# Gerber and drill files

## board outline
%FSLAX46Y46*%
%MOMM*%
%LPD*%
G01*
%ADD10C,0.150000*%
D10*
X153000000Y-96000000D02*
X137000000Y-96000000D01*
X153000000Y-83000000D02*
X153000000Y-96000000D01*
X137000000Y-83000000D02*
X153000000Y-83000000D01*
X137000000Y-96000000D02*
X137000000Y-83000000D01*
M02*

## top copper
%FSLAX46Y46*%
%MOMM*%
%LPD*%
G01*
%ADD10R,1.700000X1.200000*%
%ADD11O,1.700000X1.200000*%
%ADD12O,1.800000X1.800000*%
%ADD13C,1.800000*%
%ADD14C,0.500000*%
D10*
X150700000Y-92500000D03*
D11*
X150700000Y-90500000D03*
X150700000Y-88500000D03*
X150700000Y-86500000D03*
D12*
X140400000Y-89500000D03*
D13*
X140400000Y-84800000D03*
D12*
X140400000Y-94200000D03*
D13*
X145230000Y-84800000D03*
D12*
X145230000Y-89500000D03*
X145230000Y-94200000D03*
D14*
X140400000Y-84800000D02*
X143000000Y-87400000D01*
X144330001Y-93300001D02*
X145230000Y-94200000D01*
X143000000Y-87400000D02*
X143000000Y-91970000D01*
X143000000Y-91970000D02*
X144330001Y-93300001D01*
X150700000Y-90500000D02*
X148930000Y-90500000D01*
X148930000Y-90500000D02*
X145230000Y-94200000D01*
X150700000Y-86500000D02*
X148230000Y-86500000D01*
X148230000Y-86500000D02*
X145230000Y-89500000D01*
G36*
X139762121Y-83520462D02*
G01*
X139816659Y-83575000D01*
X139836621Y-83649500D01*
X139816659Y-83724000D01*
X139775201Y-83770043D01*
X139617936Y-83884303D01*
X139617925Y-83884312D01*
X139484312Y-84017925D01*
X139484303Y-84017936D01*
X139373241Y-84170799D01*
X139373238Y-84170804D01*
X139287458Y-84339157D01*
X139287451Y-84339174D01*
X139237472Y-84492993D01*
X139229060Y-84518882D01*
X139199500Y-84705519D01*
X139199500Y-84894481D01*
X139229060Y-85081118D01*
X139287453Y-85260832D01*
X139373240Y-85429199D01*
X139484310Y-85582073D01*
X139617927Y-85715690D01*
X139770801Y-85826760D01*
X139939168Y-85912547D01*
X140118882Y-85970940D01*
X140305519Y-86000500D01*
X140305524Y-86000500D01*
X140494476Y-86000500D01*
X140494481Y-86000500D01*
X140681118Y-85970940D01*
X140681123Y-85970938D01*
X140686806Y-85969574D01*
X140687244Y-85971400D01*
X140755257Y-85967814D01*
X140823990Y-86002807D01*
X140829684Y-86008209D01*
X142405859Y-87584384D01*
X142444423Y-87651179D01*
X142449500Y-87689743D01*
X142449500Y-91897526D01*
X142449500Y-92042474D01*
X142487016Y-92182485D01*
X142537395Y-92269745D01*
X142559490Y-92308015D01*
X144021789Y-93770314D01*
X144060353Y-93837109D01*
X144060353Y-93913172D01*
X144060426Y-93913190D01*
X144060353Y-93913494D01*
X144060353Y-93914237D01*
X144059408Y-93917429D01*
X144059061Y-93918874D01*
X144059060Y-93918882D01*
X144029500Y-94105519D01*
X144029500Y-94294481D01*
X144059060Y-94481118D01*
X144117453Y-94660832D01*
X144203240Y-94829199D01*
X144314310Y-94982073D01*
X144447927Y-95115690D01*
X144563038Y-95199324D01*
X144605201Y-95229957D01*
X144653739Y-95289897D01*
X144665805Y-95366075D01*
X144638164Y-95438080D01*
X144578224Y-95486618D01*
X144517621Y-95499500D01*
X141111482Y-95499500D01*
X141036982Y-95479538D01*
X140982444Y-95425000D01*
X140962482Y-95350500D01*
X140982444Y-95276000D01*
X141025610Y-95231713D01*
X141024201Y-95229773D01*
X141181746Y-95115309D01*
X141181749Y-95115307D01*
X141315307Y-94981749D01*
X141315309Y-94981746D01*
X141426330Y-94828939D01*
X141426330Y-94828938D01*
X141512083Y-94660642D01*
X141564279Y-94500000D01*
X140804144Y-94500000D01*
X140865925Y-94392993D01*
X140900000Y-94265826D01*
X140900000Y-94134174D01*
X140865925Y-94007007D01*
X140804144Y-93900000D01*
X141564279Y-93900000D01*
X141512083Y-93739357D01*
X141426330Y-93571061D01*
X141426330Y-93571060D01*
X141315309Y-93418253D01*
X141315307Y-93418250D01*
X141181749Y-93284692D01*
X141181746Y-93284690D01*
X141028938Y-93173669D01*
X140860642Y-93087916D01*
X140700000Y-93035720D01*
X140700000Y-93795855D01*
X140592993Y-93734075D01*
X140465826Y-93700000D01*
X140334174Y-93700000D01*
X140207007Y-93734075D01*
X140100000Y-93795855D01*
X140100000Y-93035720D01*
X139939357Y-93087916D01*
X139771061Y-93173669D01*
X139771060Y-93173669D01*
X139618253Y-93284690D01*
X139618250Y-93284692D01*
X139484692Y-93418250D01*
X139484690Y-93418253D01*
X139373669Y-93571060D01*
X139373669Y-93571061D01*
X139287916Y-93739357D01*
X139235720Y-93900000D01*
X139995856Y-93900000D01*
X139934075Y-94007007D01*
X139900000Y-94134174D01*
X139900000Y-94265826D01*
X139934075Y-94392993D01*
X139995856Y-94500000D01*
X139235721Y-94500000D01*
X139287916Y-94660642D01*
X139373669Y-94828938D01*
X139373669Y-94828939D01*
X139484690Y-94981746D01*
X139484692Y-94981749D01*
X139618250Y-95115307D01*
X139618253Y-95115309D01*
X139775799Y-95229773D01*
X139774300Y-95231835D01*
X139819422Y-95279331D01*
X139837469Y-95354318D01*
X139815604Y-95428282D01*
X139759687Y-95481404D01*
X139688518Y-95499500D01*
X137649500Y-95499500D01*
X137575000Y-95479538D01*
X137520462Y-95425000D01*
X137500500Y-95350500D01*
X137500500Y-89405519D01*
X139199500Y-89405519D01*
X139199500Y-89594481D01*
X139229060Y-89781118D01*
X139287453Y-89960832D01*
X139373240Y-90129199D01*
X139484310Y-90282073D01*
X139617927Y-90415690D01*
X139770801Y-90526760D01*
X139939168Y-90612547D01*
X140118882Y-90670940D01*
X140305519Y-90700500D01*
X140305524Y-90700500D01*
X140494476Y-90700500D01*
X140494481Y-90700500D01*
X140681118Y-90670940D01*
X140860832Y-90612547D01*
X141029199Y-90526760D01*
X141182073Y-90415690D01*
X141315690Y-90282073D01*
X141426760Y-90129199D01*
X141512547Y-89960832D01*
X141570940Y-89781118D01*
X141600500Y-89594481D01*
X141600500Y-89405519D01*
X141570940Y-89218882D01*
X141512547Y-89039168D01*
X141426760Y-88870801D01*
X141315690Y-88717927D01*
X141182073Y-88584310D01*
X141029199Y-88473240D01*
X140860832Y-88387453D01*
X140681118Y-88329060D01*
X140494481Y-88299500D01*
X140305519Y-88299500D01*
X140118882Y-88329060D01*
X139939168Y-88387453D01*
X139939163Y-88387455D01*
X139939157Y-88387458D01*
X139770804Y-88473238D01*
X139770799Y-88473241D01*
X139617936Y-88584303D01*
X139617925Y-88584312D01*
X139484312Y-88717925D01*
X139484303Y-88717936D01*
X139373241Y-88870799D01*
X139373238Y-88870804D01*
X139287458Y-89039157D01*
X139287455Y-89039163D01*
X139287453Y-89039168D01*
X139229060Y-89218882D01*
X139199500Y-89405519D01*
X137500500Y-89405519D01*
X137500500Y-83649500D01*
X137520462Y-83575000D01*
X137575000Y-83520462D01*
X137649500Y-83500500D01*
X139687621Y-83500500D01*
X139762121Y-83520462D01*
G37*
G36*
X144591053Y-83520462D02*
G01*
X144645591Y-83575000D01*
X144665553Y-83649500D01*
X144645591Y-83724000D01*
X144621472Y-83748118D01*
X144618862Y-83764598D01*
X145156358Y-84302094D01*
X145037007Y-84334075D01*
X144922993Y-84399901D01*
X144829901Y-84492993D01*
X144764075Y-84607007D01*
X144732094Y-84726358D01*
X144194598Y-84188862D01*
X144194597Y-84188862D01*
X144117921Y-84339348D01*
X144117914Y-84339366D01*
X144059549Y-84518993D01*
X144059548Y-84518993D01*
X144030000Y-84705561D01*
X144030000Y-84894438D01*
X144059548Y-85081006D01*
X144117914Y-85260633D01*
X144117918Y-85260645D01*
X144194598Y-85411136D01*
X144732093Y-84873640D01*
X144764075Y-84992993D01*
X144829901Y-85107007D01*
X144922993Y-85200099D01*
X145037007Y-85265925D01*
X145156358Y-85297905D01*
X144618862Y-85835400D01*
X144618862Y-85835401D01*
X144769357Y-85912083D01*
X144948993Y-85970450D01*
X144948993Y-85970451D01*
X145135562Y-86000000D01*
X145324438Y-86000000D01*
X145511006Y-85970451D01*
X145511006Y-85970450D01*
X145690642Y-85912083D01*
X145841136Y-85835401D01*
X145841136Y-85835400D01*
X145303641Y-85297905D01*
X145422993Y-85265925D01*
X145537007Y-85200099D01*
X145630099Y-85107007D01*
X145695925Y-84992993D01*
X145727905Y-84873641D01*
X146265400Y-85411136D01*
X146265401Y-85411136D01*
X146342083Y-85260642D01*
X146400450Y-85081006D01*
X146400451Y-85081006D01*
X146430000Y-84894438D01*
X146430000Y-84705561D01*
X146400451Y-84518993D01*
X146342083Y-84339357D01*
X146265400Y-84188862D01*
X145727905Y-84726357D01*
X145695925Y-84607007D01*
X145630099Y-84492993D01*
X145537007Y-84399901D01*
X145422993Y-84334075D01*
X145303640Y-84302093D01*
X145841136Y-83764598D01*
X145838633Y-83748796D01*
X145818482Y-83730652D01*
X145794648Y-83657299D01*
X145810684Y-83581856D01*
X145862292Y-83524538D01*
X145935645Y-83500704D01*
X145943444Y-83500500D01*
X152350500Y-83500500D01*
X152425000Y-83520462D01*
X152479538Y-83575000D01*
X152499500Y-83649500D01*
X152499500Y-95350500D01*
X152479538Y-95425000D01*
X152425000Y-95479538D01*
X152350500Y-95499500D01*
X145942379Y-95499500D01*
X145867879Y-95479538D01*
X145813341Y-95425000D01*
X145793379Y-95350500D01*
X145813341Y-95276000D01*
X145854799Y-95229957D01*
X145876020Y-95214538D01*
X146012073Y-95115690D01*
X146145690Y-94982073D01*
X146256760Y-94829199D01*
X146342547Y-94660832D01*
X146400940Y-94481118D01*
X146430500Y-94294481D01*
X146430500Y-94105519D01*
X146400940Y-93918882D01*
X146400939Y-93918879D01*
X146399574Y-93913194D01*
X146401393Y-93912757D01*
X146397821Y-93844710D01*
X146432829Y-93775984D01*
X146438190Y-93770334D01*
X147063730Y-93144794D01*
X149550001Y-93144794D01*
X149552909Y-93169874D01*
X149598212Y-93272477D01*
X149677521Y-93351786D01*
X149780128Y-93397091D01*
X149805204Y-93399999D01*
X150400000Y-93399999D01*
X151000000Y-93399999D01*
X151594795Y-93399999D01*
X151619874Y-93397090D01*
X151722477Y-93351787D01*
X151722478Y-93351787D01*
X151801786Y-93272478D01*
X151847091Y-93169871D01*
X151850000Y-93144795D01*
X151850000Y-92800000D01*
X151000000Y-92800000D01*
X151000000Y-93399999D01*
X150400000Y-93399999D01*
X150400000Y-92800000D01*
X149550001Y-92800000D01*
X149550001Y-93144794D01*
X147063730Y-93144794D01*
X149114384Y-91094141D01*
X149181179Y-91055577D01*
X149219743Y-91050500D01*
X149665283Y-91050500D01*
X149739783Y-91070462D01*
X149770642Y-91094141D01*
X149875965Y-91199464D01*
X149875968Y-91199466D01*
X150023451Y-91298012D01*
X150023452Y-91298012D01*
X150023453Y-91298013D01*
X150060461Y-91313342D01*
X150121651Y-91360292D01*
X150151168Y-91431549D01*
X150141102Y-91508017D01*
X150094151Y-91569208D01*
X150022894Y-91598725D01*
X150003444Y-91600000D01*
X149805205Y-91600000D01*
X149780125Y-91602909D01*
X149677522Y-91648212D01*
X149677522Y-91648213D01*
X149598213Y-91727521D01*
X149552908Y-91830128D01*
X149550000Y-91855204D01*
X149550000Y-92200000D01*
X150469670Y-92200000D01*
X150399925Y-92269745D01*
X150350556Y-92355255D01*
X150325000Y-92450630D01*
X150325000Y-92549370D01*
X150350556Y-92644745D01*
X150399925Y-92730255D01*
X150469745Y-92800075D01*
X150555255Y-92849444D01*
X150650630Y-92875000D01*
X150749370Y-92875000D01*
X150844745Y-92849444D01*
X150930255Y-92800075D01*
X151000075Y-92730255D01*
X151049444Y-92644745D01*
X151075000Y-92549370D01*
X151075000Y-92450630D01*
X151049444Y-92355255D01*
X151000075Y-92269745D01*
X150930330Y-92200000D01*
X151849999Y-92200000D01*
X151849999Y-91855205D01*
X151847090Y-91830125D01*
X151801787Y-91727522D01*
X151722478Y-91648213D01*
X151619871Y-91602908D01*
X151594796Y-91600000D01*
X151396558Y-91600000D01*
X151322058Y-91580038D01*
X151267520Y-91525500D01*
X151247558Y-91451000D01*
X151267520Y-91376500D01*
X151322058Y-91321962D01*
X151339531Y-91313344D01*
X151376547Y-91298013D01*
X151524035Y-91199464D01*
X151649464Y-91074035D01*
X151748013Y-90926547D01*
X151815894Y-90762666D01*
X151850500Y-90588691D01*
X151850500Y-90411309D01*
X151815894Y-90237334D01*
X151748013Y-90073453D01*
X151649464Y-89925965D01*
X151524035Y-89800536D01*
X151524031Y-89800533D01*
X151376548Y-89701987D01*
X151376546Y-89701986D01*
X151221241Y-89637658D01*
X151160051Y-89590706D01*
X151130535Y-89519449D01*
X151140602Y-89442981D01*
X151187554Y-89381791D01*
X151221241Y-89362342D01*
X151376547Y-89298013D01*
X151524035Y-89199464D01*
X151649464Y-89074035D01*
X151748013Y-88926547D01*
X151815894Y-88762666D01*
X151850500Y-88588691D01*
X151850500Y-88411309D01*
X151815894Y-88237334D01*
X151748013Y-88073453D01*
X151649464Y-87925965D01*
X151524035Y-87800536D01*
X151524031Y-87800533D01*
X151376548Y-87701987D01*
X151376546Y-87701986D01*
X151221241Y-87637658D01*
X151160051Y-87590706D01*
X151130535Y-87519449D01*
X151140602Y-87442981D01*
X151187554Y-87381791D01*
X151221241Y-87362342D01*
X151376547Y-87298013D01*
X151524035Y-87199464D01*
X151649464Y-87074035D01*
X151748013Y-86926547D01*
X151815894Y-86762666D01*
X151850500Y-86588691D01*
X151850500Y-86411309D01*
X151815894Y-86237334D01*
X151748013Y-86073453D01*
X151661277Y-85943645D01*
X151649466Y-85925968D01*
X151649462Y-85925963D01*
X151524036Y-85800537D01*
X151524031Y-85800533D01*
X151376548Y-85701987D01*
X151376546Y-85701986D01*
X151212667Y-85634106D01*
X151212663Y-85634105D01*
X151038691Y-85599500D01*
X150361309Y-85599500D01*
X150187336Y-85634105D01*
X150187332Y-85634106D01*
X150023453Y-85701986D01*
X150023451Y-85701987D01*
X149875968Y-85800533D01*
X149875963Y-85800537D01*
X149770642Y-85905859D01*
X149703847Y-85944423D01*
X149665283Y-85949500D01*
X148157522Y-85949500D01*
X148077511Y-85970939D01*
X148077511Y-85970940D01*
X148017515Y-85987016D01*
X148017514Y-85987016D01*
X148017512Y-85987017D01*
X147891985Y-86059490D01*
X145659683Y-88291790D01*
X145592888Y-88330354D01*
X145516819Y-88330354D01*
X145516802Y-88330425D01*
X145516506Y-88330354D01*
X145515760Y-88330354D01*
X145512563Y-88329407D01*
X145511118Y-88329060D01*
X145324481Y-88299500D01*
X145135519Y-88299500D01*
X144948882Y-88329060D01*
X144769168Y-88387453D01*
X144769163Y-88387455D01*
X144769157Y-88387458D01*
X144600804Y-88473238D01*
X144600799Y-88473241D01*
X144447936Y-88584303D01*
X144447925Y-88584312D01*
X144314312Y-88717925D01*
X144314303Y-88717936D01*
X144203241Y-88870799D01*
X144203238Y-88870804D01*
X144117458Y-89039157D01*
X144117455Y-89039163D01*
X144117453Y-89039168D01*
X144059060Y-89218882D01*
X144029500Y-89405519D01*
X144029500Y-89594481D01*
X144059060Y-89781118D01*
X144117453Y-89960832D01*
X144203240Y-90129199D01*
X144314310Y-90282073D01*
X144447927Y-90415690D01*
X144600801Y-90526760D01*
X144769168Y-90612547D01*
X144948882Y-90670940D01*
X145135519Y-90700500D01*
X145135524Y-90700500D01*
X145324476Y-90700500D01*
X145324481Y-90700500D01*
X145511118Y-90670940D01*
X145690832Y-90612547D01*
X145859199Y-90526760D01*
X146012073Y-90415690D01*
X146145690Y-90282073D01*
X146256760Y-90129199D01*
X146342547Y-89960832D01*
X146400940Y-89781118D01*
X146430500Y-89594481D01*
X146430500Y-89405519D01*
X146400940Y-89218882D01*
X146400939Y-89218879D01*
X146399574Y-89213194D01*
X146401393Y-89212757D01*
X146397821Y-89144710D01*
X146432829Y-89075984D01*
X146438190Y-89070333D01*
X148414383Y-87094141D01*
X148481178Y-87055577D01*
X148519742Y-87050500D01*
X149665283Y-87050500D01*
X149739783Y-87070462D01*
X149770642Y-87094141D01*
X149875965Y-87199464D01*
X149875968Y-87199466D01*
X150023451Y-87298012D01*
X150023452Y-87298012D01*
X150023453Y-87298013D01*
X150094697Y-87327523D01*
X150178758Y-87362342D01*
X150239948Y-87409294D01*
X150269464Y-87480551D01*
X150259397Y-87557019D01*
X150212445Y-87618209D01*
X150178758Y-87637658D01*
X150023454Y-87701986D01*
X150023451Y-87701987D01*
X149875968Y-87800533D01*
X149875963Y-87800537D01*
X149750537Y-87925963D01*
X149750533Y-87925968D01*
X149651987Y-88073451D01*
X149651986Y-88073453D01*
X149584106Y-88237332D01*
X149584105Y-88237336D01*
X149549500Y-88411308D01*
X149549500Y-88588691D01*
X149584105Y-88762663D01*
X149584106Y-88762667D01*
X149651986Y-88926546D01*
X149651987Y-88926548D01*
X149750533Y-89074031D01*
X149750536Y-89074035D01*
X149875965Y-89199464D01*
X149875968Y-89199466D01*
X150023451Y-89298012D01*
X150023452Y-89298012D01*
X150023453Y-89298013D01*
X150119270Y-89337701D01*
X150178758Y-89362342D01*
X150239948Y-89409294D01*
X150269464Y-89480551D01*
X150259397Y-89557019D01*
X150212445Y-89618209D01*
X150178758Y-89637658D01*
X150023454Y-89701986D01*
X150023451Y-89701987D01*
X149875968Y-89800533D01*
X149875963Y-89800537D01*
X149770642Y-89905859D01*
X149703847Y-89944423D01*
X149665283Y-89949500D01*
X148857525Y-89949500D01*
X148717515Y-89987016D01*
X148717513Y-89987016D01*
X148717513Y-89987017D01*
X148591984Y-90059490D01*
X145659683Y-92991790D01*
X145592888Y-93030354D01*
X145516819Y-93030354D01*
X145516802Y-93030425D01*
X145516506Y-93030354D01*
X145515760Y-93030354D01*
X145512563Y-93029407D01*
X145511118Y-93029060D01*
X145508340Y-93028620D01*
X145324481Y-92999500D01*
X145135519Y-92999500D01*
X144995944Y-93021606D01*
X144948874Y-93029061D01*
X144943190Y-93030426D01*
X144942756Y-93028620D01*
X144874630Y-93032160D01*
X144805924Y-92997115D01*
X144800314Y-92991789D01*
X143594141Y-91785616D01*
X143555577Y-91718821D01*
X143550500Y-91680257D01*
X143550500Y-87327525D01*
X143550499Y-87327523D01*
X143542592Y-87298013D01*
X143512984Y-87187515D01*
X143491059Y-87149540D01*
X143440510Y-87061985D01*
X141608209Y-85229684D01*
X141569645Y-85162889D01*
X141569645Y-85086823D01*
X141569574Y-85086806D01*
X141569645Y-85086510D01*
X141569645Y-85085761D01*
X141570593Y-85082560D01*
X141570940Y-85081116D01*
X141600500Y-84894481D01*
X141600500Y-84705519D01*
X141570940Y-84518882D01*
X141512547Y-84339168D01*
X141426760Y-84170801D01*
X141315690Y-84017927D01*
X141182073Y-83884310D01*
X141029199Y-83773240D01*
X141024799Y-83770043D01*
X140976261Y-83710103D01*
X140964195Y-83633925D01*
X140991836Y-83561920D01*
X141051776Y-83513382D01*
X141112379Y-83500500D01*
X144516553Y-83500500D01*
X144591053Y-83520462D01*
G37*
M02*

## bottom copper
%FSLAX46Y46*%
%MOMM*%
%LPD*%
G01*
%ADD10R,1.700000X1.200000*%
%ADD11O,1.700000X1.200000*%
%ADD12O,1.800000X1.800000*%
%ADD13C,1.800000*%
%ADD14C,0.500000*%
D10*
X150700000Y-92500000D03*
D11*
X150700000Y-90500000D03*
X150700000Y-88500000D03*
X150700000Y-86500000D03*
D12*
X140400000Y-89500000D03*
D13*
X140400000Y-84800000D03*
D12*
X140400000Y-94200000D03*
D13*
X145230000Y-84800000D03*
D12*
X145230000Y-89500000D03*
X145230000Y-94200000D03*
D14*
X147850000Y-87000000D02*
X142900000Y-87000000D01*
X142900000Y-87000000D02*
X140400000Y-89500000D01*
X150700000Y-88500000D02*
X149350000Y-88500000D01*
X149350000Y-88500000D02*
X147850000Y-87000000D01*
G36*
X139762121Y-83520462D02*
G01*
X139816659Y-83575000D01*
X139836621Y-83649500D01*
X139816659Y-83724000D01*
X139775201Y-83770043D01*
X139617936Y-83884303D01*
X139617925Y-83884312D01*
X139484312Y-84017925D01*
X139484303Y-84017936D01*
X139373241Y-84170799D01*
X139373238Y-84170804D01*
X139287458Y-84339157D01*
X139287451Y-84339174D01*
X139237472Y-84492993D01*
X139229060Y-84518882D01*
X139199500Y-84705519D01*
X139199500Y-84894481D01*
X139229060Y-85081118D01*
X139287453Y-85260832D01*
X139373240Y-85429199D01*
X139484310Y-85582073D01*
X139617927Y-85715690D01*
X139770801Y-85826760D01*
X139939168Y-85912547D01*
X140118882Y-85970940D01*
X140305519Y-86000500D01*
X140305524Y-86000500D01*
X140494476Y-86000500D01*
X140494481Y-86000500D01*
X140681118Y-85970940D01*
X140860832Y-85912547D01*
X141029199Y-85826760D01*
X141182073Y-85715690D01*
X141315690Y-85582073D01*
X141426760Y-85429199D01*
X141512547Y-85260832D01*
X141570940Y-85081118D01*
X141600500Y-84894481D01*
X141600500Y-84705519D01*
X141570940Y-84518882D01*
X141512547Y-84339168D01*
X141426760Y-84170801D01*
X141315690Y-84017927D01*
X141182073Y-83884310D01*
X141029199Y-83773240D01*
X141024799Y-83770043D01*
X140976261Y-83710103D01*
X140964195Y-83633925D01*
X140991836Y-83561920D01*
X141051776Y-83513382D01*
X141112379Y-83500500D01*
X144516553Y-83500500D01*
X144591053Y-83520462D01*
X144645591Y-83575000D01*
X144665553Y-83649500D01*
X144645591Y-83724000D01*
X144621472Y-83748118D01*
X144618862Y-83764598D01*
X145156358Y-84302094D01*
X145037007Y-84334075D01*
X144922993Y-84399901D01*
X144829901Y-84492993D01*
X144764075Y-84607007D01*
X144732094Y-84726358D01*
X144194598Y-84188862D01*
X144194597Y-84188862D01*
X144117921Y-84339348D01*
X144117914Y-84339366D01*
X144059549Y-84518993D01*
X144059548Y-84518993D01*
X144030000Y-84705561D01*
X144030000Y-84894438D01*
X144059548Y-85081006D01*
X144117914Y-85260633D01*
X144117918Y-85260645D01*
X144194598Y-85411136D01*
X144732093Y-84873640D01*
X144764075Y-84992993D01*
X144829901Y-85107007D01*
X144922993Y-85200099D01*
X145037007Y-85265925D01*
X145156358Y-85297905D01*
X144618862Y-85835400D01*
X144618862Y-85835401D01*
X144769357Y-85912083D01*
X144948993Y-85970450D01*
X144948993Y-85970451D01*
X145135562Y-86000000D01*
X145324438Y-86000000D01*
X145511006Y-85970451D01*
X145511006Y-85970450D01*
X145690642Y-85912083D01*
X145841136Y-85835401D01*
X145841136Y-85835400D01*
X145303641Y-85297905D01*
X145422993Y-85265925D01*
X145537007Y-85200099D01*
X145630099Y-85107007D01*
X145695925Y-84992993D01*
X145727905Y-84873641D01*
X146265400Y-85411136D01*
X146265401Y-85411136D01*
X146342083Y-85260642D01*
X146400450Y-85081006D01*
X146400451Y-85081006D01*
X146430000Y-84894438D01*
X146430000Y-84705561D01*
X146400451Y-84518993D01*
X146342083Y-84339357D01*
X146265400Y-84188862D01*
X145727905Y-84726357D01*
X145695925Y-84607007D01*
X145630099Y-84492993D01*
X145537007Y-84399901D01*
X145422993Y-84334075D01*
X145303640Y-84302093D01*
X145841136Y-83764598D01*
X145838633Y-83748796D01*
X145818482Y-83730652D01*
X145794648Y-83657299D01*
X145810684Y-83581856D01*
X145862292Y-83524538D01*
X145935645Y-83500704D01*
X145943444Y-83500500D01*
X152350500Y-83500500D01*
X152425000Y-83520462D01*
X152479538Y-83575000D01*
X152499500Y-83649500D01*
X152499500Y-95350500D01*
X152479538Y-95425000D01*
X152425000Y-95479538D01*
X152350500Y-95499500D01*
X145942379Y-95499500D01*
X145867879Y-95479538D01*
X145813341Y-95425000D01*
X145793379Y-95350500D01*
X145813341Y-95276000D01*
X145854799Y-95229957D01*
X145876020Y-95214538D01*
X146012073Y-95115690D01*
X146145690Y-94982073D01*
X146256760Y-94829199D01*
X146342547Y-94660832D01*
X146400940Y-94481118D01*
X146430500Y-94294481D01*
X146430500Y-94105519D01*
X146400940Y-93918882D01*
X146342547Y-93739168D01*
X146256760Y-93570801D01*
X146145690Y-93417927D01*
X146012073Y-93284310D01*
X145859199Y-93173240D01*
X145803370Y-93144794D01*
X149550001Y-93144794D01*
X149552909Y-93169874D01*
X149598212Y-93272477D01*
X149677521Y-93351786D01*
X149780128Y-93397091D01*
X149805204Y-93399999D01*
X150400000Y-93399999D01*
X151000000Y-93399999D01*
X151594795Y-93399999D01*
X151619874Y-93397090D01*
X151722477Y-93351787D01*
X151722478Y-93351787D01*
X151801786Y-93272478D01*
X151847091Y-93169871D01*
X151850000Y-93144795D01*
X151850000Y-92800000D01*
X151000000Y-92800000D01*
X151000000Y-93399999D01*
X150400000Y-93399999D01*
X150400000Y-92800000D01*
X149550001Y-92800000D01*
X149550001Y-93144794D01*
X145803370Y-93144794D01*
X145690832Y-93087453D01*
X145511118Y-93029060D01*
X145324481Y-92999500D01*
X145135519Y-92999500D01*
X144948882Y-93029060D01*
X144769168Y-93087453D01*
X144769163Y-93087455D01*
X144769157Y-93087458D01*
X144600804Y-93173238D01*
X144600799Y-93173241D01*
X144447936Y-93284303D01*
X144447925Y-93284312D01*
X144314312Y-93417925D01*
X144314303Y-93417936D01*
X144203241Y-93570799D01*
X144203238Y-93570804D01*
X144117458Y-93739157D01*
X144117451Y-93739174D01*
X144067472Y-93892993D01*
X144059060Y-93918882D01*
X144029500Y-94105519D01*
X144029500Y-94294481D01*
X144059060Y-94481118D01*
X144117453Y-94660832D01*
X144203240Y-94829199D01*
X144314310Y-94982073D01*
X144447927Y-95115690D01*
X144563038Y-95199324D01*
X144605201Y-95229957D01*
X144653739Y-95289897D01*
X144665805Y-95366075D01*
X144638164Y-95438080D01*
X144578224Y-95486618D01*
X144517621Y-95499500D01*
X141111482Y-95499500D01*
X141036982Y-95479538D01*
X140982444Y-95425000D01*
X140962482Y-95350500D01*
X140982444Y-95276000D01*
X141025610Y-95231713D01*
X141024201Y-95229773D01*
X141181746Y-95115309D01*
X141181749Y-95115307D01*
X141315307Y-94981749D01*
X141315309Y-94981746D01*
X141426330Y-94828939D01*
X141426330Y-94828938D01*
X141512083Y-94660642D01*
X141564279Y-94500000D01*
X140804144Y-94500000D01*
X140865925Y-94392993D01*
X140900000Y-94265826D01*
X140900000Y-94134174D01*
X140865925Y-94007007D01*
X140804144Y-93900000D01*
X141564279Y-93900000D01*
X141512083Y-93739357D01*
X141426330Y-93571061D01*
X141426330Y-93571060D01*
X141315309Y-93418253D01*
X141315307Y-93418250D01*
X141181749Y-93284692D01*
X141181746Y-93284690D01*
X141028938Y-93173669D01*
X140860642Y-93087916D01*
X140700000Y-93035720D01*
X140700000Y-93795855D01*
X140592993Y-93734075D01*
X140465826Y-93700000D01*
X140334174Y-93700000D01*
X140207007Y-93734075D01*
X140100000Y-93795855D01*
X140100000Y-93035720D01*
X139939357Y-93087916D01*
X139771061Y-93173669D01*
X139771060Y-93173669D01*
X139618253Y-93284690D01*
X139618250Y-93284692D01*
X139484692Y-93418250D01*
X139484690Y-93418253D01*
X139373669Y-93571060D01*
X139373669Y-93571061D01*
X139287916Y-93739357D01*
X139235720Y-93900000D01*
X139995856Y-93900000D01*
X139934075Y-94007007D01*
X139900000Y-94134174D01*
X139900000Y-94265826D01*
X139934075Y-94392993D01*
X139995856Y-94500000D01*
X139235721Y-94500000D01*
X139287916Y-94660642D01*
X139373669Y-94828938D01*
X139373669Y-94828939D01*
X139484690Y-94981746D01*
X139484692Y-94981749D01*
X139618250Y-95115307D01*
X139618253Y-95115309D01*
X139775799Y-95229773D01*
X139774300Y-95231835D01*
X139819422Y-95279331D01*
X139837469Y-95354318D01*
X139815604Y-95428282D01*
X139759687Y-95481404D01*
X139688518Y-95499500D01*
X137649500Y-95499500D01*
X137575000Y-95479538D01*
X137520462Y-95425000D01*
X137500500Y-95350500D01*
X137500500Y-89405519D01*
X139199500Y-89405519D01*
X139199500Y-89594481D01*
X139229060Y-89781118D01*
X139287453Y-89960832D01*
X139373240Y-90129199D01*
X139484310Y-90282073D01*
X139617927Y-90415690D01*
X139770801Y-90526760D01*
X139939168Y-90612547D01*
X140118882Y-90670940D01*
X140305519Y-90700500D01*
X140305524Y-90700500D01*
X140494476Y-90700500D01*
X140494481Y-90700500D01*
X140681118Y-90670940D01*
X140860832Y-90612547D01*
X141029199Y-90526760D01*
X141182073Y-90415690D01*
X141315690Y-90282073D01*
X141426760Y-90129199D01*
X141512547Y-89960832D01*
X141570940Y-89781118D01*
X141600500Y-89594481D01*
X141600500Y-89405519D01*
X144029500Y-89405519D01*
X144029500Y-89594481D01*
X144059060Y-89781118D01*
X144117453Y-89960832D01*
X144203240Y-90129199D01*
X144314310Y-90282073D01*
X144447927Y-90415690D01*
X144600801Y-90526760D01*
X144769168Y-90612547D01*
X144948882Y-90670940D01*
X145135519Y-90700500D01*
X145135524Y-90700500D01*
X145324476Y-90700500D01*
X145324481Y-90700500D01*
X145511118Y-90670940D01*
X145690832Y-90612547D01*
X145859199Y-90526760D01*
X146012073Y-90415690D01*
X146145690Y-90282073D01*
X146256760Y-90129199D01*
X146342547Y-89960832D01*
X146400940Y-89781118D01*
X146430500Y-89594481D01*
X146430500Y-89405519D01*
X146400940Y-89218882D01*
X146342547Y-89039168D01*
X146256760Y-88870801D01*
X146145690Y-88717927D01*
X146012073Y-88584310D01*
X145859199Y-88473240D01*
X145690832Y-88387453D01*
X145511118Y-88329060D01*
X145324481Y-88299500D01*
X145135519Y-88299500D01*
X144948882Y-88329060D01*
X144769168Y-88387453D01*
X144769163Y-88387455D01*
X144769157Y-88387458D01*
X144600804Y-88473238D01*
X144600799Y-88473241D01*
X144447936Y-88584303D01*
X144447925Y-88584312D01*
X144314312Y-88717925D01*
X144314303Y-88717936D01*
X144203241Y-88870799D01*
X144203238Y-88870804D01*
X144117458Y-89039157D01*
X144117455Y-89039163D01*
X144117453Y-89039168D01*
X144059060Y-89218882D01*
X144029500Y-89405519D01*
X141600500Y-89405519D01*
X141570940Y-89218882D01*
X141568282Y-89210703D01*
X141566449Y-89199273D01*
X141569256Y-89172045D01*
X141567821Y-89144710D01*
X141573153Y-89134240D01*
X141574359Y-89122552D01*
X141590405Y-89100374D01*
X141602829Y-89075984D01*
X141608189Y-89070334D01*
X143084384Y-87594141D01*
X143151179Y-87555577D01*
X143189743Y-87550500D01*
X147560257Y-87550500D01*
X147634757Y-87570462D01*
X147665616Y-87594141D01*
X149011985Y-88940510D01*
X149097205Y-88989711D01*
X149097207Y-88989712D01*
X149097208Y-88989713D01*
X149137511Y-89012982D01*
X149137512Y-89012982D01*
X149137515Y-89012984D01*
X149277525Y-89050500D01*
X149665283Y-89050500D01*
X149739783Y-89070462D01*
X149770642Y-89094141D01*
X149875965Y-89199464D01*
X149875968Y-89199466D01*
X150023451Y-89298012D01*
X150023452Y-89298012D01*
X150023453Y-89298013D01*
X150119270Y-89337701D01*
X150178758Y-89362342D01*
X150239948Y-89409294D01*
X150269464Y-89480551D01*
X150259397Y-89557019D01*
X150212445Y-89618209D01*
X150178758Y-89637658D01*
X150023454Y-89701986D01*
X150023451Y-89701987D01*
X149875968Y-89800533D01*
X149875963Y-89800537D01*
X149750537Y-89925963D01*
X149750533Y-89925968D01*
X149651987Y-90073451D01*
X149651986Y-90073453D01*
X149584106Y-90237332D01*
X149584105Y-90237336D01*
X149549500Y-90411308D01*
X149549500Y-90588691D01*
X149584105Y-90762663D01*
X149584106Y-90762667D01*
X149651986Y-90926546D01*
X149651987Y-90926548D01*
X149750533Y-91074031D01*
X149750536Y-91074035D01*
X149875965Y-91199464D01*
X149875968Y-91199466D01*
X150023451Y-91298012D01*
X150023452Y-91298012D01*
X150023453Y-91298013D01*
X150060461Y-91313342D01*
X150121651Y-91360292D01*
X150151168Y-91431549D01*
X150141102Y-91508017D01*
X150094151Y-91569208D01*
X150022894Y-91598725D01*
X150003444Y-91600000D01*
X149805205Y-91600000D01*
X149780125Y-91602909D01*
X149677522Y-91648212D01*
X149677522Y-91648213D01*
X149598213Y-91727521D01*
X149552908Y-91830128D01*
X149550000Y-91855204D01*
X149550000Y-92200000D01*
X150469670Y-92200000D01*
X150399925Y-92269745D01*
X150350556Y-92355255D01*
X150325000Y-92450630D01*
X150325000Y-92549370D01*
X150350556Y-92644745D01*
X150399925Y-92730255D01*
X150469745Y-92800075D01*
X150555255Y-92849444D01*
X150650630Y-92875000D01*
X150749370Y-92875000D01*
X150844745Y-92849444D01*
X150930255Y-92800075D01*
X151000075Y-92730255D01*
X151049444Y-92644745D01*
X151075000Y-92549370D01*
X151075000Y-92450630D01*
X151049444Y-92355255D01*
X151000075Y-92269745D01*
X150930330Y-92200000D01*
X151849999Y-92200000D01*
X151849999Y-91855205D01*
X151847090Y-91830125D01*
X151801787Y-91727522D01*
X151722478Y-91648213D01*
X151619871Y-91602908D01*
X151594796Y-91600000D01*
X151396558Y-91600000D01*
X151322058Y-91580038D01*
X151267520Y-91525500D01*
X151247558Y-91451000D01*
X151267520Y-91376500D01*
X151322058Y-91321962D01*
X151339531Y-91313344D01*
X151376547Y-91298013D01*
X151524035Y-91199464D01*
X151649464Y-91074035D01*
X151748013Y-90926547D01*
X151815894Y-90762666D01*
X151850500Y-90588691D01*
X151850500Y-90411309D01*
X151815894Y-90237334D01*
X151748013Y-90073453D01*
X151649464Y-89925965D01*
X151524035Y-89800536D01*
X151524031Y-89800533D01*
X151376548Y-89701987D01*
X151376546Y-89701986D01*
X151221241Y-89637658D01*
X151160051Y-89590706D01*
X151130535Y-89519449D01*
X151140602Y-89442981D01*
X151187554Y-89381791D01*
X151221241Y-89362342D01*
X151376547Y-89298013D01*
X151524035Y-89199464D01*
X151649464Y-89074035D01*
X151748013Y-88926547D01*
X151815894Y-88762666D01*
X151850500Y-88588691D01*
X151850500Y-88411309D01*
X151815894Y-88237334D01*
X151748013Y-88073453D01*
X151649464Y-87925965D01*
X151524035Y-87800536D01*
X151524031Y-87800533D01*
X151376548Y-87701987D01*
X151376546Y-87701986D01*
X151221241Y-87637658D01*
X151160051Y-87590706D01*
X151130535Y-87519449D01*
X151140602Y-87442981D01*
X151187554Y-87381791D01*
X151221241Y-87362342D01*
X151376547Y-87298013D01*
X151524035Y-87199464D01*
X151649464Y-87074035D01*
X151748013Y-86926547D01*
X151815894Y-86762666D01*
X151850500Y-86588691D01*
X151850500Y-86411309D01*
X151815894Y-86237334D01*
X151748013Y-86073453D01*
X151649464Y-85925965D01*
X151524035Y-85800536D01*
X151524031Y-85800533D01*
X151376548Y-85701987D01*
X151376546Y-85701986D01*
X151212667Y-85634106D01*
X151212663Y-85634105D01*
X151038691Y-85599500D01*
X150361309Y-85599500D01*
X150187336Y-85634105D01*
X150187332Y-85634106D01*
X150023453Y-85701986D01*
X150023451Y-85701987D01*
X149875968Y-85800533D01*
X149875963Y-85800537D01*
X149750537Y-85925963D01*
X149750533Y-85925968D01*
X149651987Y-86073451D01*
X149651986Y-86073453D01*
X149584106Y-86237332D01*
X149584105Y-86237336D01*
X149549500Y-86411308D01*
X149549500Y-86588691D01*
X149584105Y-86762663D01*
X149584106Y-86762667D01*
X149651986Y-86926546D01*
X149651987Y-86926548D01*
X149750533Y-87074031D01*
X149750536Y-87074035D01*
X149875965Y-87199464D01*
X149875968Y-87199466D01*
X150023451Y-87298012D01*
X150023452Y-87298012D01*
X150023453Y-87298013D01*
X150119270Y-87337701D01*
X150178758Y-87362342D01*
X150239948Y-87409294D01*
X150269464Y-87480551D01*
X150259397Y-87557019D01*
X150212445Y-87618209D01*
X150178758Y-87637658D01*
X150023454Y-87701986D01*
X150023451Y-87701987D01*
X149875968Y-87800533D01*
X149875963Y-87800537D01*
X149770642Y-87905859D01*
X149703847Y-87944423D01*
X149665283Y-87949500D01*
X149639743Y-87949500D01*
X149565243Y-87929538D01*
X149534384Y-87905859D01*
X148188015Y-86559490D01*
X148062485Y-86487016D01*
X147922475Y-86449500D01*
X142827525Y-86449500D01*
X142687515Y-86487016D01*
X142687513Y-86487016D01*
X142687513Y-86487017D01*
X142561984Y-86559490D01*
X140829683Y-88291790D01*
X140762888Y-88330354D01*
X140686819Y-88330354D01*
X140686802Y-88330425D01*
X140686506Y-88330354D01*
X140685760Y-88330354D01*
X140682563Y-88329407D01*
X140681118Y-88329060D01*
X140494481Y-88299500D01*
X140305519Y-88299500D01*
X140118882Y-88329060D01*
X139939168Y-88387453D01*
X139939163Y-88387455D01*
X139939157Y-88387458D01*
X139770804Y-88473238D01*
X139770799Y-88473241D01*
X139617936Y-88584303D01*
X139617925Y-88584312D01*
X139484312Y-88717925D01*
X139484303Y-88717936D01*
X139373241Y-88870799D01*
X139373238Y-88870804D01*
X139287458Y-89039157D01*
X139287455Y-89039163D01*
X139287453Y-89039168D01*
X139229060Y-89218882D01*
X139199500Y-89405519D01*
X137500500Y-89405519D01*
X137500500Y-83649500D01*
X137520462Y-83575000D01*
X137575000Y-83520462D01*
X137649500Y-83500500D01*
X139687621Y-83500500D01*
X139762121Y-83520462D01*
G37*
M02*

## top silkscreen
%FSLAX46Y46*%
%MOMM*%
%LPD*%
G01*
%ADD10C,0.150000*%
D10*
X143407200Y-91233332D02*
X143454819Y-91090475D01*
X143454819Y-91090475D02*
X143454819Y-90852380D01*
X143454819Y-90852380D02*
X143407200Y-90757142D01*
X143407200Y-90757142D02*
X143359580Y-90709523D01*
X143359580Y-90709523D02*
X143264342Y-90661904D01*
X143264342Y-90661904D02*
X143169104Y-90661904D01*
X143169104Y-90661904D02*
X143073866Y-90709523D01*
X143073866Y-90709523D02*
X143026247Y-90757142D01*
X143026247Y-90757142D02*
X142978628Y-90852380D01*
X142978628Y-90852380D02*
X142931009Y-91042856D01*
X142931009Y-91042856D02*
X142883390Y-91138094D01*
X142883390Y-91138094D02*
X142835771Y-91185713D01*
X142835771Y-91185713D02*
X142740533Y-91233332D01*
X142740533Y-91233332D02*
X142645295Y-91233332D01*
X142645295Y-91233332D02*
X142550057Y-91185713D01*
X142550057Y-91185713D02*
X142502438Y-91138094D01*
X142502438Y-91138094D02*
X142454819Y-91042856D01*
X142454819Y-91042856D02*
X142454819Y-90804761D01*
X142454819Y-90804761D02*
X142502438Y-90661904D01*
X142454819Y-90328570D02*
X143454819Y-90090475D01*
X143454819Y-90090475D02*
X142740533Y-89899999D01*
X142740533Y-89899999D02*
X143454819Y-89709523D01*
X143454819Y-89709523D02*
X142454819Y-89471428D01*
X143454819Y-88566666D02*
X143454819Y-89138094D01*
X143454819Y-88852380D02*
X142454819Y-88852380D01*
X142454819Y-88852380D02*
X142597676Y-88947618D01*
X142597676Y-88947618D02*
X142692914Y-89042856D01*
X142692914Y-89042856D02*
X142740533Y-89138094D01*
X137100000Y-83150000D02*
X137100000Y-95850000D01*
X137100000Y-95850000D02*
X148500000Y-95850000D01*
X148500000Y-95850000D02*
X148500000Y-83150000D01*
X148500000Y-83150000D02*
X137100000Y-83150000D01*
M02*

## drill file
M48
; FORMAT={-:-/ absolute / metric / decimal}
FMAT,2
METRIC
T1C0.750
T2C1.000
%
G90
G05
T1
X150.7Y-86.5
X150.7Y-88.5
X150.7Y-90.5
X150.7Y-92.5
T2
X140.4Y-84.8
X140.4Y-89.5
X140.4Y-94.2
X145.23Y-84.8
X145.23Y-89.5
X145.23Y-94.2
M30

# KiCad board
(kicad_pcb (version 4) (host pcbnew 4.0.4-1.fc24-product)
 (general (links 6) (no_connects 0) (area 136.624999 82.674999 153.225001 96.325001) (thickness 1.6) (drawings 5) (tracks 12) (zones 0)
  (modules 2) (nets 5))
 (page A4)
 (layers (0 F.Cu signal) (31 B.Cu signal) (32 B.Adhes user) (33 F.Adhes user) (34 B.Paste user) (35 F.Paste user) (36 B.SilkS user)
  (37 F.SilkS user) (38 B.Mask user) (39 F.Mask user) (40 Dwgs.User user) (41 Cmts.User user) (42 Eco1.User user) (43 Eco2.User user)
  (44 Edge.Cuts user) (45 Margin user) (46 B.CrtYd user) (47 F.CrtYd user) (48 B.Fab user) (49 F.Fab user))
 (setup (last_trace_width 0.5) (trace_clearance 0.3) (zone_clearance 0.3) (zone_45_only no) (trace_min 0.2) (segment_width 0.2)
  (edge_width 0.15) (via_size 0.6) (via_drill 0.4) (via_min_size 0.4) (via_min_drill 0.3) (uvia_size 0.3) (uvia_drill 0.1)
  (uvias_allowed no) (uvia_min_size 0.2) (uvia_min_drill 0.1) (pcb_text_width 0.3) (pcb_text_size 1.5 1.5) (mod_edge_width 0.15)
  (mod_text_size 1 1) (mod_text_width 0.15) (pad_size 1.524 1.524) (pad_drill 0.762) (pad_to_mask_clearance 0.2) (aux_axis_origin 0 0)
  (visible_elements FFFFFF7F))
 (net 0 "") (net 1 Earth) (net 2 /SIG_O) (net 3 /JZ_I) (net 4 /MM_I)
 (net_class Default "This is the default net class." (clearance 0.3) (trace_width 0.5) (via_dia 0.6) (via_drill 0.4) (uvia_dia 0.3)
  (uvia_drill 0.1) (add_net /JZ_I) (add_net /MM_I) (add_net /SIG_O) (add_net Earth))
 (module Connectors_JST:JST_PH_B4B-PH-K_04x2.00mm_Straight (layer B.Cu) (at 150.7 92.5 90)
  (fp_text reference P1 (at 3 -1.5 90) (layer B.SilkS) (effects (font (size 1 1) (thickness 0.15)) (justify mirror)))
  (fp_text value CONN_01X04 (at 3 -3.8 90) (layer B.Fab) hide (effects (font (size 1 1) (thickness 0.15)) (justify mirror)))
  (pad 1 thru_hole rect (at 0 0 90) (size 1.2 1.7) (drill 0.75) (layers *.Cu *.Mask) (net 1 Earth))
  (pad 2 thru_hole oval (at 2 0 90) (size 1.2 1.7) (drill 0.75) (layers *.Cu *.Mask) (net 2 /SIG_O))
  (pad 3 thru_hole oval (at 4 0 90) (size 1.2 1.7) (drill 0.75) (layers *.Cu *.Mask) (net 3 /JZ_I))
  (pad 4 thru_hole oval (at 6 0 90) (size 1.2 1.7) (drill 0.75) (layers *.Cu *.Mask) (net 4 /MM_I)))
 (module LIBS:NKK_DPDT (layer F.Cu) (at 145.2 84.8 90)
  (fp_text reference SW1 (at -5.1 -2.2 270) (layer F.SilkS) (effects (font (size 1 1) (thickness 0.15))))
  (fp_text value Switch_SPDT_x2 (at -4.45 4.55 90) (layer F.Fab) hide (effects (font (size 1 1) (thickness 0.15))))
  (fp_line (start 1.65 -8.1) (end -11.05 -8.1) (layer F.SilkS) (width 0.15))
  (fp_line (start -11.05 -8.1) (end -11.05 3.3) (layer F.SilkS) (width 0.15))
  (fp_line (start -11.05 3.3) (end 1.65 3.3) (layer F.SilkS) (width 0.15))
  (fp_line (start 1.65 3.3) (end 1.65 -8.1) (layer F.SilkS) (width 0.15))
  (pad 5 thru_hole oval (at -4.7 -4.8 270) (size 1.8 1.8) (drill 1) (layers *.Cu *.Mask) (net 3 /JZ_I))
  (pad 4 thru_hole circle (at 0 -4.8 270) (size 1.8 1.8) (drill 1) (layers *.Cu *.Mask) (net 2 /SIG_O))
  (pad 6 thru_hole oval (at -9.4 -4.8 270) (size 1.8 1.8) (drill 1) (layers *.Cu *.Mask) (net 1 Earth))
  (pad 1 thru_hole circle (at 0 0.03 270) (size 1.8 1.8) (drill 1) (layers *.Cu *.Mask) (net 1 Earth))
  (pad 2 thru_hole oval (at -4.7 0.03 270) (size 1.8 1.8) (drill 1) (layers *.Cu *.Mask) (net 4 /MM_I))
  (pad 3 thru_hole oval (at -9.4 0.03 270) (size 1.8 1.8) (drill 1) (layers *.Cu *.Mask) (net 2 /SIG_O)))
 (gr_line (start 153 96) (end 137 96) (layer Edge.Cuts) (width 0.15))
 (gr_line (start 153 83) (end 153 96) (layer Edge.Cuts) (width 0.15))
 (gr_line (start 137 83) (end 153 83) (layer Edge.Cuts) (width 0.15))
 (gr_line (start 137 96) (end 137 83) (layer Edge.Cuts) (width 0.15))
 (segment (start 140.4 84.8) (end 143 87.4) (width 0.5) (layer F.Cu) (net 2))
 (segment (start 144.330001 93.300001) (end 145.23 94.2) (width 0.5) (layer F.Cu) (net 2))
 (segment (start 143 87.4) (end 143 91.97) (width 0.5) (layer F.Cu) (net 2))
 (segment (start 143 91.97) (end 144.330001 93.300001) (width 0.5) (layer F.Cu) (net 2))
 (segment (start 150.7 90.5) (end 148.93 90.5) (width 0.5) (layer F.Cu) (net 2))
 (segment (start 148.93 90.5) (end 145.23 94.2) (width 0.5) (layer F.Cu) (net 2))
 (segment (start 147.85 87) (end 142.9 87) (width 0.5) (layer B.Cu) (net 3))
 (segment (start 142.9 87) (end 140.4 89.5) (width 0.5) (layer B.Cu) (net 3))
 (segment (start 150.7 88.5) (end 149.35 88.5) (width 0.5) (layer B.Cu) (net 3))
 (segment (start 149.35 88.5) (end 147.85 87) (width 0.5) (layer B.Cu) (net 3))
 (segment (start 150.7 86.5) (end 148.23 86.5) (width 0.5) (layer F.Cu) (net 4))
 (segment (start 148.23 86.5) (end 145.23 89.5) (width 0.5) (layer F.Cu) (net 4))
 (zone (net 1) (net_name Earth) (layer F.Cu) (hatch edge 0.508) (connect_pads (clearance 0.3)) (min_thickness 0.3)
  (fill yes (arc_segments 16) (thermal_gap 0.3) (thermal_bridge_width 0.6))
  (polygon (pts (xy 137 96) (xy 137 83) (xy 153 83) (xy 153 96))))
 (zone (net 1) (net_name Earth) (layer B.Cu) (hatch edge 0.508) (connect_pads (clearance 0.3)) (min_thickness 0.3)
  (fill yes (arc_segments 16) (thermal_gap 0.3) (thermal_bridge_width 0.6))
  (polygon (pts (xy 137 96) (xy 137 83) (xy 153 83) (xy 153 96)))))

